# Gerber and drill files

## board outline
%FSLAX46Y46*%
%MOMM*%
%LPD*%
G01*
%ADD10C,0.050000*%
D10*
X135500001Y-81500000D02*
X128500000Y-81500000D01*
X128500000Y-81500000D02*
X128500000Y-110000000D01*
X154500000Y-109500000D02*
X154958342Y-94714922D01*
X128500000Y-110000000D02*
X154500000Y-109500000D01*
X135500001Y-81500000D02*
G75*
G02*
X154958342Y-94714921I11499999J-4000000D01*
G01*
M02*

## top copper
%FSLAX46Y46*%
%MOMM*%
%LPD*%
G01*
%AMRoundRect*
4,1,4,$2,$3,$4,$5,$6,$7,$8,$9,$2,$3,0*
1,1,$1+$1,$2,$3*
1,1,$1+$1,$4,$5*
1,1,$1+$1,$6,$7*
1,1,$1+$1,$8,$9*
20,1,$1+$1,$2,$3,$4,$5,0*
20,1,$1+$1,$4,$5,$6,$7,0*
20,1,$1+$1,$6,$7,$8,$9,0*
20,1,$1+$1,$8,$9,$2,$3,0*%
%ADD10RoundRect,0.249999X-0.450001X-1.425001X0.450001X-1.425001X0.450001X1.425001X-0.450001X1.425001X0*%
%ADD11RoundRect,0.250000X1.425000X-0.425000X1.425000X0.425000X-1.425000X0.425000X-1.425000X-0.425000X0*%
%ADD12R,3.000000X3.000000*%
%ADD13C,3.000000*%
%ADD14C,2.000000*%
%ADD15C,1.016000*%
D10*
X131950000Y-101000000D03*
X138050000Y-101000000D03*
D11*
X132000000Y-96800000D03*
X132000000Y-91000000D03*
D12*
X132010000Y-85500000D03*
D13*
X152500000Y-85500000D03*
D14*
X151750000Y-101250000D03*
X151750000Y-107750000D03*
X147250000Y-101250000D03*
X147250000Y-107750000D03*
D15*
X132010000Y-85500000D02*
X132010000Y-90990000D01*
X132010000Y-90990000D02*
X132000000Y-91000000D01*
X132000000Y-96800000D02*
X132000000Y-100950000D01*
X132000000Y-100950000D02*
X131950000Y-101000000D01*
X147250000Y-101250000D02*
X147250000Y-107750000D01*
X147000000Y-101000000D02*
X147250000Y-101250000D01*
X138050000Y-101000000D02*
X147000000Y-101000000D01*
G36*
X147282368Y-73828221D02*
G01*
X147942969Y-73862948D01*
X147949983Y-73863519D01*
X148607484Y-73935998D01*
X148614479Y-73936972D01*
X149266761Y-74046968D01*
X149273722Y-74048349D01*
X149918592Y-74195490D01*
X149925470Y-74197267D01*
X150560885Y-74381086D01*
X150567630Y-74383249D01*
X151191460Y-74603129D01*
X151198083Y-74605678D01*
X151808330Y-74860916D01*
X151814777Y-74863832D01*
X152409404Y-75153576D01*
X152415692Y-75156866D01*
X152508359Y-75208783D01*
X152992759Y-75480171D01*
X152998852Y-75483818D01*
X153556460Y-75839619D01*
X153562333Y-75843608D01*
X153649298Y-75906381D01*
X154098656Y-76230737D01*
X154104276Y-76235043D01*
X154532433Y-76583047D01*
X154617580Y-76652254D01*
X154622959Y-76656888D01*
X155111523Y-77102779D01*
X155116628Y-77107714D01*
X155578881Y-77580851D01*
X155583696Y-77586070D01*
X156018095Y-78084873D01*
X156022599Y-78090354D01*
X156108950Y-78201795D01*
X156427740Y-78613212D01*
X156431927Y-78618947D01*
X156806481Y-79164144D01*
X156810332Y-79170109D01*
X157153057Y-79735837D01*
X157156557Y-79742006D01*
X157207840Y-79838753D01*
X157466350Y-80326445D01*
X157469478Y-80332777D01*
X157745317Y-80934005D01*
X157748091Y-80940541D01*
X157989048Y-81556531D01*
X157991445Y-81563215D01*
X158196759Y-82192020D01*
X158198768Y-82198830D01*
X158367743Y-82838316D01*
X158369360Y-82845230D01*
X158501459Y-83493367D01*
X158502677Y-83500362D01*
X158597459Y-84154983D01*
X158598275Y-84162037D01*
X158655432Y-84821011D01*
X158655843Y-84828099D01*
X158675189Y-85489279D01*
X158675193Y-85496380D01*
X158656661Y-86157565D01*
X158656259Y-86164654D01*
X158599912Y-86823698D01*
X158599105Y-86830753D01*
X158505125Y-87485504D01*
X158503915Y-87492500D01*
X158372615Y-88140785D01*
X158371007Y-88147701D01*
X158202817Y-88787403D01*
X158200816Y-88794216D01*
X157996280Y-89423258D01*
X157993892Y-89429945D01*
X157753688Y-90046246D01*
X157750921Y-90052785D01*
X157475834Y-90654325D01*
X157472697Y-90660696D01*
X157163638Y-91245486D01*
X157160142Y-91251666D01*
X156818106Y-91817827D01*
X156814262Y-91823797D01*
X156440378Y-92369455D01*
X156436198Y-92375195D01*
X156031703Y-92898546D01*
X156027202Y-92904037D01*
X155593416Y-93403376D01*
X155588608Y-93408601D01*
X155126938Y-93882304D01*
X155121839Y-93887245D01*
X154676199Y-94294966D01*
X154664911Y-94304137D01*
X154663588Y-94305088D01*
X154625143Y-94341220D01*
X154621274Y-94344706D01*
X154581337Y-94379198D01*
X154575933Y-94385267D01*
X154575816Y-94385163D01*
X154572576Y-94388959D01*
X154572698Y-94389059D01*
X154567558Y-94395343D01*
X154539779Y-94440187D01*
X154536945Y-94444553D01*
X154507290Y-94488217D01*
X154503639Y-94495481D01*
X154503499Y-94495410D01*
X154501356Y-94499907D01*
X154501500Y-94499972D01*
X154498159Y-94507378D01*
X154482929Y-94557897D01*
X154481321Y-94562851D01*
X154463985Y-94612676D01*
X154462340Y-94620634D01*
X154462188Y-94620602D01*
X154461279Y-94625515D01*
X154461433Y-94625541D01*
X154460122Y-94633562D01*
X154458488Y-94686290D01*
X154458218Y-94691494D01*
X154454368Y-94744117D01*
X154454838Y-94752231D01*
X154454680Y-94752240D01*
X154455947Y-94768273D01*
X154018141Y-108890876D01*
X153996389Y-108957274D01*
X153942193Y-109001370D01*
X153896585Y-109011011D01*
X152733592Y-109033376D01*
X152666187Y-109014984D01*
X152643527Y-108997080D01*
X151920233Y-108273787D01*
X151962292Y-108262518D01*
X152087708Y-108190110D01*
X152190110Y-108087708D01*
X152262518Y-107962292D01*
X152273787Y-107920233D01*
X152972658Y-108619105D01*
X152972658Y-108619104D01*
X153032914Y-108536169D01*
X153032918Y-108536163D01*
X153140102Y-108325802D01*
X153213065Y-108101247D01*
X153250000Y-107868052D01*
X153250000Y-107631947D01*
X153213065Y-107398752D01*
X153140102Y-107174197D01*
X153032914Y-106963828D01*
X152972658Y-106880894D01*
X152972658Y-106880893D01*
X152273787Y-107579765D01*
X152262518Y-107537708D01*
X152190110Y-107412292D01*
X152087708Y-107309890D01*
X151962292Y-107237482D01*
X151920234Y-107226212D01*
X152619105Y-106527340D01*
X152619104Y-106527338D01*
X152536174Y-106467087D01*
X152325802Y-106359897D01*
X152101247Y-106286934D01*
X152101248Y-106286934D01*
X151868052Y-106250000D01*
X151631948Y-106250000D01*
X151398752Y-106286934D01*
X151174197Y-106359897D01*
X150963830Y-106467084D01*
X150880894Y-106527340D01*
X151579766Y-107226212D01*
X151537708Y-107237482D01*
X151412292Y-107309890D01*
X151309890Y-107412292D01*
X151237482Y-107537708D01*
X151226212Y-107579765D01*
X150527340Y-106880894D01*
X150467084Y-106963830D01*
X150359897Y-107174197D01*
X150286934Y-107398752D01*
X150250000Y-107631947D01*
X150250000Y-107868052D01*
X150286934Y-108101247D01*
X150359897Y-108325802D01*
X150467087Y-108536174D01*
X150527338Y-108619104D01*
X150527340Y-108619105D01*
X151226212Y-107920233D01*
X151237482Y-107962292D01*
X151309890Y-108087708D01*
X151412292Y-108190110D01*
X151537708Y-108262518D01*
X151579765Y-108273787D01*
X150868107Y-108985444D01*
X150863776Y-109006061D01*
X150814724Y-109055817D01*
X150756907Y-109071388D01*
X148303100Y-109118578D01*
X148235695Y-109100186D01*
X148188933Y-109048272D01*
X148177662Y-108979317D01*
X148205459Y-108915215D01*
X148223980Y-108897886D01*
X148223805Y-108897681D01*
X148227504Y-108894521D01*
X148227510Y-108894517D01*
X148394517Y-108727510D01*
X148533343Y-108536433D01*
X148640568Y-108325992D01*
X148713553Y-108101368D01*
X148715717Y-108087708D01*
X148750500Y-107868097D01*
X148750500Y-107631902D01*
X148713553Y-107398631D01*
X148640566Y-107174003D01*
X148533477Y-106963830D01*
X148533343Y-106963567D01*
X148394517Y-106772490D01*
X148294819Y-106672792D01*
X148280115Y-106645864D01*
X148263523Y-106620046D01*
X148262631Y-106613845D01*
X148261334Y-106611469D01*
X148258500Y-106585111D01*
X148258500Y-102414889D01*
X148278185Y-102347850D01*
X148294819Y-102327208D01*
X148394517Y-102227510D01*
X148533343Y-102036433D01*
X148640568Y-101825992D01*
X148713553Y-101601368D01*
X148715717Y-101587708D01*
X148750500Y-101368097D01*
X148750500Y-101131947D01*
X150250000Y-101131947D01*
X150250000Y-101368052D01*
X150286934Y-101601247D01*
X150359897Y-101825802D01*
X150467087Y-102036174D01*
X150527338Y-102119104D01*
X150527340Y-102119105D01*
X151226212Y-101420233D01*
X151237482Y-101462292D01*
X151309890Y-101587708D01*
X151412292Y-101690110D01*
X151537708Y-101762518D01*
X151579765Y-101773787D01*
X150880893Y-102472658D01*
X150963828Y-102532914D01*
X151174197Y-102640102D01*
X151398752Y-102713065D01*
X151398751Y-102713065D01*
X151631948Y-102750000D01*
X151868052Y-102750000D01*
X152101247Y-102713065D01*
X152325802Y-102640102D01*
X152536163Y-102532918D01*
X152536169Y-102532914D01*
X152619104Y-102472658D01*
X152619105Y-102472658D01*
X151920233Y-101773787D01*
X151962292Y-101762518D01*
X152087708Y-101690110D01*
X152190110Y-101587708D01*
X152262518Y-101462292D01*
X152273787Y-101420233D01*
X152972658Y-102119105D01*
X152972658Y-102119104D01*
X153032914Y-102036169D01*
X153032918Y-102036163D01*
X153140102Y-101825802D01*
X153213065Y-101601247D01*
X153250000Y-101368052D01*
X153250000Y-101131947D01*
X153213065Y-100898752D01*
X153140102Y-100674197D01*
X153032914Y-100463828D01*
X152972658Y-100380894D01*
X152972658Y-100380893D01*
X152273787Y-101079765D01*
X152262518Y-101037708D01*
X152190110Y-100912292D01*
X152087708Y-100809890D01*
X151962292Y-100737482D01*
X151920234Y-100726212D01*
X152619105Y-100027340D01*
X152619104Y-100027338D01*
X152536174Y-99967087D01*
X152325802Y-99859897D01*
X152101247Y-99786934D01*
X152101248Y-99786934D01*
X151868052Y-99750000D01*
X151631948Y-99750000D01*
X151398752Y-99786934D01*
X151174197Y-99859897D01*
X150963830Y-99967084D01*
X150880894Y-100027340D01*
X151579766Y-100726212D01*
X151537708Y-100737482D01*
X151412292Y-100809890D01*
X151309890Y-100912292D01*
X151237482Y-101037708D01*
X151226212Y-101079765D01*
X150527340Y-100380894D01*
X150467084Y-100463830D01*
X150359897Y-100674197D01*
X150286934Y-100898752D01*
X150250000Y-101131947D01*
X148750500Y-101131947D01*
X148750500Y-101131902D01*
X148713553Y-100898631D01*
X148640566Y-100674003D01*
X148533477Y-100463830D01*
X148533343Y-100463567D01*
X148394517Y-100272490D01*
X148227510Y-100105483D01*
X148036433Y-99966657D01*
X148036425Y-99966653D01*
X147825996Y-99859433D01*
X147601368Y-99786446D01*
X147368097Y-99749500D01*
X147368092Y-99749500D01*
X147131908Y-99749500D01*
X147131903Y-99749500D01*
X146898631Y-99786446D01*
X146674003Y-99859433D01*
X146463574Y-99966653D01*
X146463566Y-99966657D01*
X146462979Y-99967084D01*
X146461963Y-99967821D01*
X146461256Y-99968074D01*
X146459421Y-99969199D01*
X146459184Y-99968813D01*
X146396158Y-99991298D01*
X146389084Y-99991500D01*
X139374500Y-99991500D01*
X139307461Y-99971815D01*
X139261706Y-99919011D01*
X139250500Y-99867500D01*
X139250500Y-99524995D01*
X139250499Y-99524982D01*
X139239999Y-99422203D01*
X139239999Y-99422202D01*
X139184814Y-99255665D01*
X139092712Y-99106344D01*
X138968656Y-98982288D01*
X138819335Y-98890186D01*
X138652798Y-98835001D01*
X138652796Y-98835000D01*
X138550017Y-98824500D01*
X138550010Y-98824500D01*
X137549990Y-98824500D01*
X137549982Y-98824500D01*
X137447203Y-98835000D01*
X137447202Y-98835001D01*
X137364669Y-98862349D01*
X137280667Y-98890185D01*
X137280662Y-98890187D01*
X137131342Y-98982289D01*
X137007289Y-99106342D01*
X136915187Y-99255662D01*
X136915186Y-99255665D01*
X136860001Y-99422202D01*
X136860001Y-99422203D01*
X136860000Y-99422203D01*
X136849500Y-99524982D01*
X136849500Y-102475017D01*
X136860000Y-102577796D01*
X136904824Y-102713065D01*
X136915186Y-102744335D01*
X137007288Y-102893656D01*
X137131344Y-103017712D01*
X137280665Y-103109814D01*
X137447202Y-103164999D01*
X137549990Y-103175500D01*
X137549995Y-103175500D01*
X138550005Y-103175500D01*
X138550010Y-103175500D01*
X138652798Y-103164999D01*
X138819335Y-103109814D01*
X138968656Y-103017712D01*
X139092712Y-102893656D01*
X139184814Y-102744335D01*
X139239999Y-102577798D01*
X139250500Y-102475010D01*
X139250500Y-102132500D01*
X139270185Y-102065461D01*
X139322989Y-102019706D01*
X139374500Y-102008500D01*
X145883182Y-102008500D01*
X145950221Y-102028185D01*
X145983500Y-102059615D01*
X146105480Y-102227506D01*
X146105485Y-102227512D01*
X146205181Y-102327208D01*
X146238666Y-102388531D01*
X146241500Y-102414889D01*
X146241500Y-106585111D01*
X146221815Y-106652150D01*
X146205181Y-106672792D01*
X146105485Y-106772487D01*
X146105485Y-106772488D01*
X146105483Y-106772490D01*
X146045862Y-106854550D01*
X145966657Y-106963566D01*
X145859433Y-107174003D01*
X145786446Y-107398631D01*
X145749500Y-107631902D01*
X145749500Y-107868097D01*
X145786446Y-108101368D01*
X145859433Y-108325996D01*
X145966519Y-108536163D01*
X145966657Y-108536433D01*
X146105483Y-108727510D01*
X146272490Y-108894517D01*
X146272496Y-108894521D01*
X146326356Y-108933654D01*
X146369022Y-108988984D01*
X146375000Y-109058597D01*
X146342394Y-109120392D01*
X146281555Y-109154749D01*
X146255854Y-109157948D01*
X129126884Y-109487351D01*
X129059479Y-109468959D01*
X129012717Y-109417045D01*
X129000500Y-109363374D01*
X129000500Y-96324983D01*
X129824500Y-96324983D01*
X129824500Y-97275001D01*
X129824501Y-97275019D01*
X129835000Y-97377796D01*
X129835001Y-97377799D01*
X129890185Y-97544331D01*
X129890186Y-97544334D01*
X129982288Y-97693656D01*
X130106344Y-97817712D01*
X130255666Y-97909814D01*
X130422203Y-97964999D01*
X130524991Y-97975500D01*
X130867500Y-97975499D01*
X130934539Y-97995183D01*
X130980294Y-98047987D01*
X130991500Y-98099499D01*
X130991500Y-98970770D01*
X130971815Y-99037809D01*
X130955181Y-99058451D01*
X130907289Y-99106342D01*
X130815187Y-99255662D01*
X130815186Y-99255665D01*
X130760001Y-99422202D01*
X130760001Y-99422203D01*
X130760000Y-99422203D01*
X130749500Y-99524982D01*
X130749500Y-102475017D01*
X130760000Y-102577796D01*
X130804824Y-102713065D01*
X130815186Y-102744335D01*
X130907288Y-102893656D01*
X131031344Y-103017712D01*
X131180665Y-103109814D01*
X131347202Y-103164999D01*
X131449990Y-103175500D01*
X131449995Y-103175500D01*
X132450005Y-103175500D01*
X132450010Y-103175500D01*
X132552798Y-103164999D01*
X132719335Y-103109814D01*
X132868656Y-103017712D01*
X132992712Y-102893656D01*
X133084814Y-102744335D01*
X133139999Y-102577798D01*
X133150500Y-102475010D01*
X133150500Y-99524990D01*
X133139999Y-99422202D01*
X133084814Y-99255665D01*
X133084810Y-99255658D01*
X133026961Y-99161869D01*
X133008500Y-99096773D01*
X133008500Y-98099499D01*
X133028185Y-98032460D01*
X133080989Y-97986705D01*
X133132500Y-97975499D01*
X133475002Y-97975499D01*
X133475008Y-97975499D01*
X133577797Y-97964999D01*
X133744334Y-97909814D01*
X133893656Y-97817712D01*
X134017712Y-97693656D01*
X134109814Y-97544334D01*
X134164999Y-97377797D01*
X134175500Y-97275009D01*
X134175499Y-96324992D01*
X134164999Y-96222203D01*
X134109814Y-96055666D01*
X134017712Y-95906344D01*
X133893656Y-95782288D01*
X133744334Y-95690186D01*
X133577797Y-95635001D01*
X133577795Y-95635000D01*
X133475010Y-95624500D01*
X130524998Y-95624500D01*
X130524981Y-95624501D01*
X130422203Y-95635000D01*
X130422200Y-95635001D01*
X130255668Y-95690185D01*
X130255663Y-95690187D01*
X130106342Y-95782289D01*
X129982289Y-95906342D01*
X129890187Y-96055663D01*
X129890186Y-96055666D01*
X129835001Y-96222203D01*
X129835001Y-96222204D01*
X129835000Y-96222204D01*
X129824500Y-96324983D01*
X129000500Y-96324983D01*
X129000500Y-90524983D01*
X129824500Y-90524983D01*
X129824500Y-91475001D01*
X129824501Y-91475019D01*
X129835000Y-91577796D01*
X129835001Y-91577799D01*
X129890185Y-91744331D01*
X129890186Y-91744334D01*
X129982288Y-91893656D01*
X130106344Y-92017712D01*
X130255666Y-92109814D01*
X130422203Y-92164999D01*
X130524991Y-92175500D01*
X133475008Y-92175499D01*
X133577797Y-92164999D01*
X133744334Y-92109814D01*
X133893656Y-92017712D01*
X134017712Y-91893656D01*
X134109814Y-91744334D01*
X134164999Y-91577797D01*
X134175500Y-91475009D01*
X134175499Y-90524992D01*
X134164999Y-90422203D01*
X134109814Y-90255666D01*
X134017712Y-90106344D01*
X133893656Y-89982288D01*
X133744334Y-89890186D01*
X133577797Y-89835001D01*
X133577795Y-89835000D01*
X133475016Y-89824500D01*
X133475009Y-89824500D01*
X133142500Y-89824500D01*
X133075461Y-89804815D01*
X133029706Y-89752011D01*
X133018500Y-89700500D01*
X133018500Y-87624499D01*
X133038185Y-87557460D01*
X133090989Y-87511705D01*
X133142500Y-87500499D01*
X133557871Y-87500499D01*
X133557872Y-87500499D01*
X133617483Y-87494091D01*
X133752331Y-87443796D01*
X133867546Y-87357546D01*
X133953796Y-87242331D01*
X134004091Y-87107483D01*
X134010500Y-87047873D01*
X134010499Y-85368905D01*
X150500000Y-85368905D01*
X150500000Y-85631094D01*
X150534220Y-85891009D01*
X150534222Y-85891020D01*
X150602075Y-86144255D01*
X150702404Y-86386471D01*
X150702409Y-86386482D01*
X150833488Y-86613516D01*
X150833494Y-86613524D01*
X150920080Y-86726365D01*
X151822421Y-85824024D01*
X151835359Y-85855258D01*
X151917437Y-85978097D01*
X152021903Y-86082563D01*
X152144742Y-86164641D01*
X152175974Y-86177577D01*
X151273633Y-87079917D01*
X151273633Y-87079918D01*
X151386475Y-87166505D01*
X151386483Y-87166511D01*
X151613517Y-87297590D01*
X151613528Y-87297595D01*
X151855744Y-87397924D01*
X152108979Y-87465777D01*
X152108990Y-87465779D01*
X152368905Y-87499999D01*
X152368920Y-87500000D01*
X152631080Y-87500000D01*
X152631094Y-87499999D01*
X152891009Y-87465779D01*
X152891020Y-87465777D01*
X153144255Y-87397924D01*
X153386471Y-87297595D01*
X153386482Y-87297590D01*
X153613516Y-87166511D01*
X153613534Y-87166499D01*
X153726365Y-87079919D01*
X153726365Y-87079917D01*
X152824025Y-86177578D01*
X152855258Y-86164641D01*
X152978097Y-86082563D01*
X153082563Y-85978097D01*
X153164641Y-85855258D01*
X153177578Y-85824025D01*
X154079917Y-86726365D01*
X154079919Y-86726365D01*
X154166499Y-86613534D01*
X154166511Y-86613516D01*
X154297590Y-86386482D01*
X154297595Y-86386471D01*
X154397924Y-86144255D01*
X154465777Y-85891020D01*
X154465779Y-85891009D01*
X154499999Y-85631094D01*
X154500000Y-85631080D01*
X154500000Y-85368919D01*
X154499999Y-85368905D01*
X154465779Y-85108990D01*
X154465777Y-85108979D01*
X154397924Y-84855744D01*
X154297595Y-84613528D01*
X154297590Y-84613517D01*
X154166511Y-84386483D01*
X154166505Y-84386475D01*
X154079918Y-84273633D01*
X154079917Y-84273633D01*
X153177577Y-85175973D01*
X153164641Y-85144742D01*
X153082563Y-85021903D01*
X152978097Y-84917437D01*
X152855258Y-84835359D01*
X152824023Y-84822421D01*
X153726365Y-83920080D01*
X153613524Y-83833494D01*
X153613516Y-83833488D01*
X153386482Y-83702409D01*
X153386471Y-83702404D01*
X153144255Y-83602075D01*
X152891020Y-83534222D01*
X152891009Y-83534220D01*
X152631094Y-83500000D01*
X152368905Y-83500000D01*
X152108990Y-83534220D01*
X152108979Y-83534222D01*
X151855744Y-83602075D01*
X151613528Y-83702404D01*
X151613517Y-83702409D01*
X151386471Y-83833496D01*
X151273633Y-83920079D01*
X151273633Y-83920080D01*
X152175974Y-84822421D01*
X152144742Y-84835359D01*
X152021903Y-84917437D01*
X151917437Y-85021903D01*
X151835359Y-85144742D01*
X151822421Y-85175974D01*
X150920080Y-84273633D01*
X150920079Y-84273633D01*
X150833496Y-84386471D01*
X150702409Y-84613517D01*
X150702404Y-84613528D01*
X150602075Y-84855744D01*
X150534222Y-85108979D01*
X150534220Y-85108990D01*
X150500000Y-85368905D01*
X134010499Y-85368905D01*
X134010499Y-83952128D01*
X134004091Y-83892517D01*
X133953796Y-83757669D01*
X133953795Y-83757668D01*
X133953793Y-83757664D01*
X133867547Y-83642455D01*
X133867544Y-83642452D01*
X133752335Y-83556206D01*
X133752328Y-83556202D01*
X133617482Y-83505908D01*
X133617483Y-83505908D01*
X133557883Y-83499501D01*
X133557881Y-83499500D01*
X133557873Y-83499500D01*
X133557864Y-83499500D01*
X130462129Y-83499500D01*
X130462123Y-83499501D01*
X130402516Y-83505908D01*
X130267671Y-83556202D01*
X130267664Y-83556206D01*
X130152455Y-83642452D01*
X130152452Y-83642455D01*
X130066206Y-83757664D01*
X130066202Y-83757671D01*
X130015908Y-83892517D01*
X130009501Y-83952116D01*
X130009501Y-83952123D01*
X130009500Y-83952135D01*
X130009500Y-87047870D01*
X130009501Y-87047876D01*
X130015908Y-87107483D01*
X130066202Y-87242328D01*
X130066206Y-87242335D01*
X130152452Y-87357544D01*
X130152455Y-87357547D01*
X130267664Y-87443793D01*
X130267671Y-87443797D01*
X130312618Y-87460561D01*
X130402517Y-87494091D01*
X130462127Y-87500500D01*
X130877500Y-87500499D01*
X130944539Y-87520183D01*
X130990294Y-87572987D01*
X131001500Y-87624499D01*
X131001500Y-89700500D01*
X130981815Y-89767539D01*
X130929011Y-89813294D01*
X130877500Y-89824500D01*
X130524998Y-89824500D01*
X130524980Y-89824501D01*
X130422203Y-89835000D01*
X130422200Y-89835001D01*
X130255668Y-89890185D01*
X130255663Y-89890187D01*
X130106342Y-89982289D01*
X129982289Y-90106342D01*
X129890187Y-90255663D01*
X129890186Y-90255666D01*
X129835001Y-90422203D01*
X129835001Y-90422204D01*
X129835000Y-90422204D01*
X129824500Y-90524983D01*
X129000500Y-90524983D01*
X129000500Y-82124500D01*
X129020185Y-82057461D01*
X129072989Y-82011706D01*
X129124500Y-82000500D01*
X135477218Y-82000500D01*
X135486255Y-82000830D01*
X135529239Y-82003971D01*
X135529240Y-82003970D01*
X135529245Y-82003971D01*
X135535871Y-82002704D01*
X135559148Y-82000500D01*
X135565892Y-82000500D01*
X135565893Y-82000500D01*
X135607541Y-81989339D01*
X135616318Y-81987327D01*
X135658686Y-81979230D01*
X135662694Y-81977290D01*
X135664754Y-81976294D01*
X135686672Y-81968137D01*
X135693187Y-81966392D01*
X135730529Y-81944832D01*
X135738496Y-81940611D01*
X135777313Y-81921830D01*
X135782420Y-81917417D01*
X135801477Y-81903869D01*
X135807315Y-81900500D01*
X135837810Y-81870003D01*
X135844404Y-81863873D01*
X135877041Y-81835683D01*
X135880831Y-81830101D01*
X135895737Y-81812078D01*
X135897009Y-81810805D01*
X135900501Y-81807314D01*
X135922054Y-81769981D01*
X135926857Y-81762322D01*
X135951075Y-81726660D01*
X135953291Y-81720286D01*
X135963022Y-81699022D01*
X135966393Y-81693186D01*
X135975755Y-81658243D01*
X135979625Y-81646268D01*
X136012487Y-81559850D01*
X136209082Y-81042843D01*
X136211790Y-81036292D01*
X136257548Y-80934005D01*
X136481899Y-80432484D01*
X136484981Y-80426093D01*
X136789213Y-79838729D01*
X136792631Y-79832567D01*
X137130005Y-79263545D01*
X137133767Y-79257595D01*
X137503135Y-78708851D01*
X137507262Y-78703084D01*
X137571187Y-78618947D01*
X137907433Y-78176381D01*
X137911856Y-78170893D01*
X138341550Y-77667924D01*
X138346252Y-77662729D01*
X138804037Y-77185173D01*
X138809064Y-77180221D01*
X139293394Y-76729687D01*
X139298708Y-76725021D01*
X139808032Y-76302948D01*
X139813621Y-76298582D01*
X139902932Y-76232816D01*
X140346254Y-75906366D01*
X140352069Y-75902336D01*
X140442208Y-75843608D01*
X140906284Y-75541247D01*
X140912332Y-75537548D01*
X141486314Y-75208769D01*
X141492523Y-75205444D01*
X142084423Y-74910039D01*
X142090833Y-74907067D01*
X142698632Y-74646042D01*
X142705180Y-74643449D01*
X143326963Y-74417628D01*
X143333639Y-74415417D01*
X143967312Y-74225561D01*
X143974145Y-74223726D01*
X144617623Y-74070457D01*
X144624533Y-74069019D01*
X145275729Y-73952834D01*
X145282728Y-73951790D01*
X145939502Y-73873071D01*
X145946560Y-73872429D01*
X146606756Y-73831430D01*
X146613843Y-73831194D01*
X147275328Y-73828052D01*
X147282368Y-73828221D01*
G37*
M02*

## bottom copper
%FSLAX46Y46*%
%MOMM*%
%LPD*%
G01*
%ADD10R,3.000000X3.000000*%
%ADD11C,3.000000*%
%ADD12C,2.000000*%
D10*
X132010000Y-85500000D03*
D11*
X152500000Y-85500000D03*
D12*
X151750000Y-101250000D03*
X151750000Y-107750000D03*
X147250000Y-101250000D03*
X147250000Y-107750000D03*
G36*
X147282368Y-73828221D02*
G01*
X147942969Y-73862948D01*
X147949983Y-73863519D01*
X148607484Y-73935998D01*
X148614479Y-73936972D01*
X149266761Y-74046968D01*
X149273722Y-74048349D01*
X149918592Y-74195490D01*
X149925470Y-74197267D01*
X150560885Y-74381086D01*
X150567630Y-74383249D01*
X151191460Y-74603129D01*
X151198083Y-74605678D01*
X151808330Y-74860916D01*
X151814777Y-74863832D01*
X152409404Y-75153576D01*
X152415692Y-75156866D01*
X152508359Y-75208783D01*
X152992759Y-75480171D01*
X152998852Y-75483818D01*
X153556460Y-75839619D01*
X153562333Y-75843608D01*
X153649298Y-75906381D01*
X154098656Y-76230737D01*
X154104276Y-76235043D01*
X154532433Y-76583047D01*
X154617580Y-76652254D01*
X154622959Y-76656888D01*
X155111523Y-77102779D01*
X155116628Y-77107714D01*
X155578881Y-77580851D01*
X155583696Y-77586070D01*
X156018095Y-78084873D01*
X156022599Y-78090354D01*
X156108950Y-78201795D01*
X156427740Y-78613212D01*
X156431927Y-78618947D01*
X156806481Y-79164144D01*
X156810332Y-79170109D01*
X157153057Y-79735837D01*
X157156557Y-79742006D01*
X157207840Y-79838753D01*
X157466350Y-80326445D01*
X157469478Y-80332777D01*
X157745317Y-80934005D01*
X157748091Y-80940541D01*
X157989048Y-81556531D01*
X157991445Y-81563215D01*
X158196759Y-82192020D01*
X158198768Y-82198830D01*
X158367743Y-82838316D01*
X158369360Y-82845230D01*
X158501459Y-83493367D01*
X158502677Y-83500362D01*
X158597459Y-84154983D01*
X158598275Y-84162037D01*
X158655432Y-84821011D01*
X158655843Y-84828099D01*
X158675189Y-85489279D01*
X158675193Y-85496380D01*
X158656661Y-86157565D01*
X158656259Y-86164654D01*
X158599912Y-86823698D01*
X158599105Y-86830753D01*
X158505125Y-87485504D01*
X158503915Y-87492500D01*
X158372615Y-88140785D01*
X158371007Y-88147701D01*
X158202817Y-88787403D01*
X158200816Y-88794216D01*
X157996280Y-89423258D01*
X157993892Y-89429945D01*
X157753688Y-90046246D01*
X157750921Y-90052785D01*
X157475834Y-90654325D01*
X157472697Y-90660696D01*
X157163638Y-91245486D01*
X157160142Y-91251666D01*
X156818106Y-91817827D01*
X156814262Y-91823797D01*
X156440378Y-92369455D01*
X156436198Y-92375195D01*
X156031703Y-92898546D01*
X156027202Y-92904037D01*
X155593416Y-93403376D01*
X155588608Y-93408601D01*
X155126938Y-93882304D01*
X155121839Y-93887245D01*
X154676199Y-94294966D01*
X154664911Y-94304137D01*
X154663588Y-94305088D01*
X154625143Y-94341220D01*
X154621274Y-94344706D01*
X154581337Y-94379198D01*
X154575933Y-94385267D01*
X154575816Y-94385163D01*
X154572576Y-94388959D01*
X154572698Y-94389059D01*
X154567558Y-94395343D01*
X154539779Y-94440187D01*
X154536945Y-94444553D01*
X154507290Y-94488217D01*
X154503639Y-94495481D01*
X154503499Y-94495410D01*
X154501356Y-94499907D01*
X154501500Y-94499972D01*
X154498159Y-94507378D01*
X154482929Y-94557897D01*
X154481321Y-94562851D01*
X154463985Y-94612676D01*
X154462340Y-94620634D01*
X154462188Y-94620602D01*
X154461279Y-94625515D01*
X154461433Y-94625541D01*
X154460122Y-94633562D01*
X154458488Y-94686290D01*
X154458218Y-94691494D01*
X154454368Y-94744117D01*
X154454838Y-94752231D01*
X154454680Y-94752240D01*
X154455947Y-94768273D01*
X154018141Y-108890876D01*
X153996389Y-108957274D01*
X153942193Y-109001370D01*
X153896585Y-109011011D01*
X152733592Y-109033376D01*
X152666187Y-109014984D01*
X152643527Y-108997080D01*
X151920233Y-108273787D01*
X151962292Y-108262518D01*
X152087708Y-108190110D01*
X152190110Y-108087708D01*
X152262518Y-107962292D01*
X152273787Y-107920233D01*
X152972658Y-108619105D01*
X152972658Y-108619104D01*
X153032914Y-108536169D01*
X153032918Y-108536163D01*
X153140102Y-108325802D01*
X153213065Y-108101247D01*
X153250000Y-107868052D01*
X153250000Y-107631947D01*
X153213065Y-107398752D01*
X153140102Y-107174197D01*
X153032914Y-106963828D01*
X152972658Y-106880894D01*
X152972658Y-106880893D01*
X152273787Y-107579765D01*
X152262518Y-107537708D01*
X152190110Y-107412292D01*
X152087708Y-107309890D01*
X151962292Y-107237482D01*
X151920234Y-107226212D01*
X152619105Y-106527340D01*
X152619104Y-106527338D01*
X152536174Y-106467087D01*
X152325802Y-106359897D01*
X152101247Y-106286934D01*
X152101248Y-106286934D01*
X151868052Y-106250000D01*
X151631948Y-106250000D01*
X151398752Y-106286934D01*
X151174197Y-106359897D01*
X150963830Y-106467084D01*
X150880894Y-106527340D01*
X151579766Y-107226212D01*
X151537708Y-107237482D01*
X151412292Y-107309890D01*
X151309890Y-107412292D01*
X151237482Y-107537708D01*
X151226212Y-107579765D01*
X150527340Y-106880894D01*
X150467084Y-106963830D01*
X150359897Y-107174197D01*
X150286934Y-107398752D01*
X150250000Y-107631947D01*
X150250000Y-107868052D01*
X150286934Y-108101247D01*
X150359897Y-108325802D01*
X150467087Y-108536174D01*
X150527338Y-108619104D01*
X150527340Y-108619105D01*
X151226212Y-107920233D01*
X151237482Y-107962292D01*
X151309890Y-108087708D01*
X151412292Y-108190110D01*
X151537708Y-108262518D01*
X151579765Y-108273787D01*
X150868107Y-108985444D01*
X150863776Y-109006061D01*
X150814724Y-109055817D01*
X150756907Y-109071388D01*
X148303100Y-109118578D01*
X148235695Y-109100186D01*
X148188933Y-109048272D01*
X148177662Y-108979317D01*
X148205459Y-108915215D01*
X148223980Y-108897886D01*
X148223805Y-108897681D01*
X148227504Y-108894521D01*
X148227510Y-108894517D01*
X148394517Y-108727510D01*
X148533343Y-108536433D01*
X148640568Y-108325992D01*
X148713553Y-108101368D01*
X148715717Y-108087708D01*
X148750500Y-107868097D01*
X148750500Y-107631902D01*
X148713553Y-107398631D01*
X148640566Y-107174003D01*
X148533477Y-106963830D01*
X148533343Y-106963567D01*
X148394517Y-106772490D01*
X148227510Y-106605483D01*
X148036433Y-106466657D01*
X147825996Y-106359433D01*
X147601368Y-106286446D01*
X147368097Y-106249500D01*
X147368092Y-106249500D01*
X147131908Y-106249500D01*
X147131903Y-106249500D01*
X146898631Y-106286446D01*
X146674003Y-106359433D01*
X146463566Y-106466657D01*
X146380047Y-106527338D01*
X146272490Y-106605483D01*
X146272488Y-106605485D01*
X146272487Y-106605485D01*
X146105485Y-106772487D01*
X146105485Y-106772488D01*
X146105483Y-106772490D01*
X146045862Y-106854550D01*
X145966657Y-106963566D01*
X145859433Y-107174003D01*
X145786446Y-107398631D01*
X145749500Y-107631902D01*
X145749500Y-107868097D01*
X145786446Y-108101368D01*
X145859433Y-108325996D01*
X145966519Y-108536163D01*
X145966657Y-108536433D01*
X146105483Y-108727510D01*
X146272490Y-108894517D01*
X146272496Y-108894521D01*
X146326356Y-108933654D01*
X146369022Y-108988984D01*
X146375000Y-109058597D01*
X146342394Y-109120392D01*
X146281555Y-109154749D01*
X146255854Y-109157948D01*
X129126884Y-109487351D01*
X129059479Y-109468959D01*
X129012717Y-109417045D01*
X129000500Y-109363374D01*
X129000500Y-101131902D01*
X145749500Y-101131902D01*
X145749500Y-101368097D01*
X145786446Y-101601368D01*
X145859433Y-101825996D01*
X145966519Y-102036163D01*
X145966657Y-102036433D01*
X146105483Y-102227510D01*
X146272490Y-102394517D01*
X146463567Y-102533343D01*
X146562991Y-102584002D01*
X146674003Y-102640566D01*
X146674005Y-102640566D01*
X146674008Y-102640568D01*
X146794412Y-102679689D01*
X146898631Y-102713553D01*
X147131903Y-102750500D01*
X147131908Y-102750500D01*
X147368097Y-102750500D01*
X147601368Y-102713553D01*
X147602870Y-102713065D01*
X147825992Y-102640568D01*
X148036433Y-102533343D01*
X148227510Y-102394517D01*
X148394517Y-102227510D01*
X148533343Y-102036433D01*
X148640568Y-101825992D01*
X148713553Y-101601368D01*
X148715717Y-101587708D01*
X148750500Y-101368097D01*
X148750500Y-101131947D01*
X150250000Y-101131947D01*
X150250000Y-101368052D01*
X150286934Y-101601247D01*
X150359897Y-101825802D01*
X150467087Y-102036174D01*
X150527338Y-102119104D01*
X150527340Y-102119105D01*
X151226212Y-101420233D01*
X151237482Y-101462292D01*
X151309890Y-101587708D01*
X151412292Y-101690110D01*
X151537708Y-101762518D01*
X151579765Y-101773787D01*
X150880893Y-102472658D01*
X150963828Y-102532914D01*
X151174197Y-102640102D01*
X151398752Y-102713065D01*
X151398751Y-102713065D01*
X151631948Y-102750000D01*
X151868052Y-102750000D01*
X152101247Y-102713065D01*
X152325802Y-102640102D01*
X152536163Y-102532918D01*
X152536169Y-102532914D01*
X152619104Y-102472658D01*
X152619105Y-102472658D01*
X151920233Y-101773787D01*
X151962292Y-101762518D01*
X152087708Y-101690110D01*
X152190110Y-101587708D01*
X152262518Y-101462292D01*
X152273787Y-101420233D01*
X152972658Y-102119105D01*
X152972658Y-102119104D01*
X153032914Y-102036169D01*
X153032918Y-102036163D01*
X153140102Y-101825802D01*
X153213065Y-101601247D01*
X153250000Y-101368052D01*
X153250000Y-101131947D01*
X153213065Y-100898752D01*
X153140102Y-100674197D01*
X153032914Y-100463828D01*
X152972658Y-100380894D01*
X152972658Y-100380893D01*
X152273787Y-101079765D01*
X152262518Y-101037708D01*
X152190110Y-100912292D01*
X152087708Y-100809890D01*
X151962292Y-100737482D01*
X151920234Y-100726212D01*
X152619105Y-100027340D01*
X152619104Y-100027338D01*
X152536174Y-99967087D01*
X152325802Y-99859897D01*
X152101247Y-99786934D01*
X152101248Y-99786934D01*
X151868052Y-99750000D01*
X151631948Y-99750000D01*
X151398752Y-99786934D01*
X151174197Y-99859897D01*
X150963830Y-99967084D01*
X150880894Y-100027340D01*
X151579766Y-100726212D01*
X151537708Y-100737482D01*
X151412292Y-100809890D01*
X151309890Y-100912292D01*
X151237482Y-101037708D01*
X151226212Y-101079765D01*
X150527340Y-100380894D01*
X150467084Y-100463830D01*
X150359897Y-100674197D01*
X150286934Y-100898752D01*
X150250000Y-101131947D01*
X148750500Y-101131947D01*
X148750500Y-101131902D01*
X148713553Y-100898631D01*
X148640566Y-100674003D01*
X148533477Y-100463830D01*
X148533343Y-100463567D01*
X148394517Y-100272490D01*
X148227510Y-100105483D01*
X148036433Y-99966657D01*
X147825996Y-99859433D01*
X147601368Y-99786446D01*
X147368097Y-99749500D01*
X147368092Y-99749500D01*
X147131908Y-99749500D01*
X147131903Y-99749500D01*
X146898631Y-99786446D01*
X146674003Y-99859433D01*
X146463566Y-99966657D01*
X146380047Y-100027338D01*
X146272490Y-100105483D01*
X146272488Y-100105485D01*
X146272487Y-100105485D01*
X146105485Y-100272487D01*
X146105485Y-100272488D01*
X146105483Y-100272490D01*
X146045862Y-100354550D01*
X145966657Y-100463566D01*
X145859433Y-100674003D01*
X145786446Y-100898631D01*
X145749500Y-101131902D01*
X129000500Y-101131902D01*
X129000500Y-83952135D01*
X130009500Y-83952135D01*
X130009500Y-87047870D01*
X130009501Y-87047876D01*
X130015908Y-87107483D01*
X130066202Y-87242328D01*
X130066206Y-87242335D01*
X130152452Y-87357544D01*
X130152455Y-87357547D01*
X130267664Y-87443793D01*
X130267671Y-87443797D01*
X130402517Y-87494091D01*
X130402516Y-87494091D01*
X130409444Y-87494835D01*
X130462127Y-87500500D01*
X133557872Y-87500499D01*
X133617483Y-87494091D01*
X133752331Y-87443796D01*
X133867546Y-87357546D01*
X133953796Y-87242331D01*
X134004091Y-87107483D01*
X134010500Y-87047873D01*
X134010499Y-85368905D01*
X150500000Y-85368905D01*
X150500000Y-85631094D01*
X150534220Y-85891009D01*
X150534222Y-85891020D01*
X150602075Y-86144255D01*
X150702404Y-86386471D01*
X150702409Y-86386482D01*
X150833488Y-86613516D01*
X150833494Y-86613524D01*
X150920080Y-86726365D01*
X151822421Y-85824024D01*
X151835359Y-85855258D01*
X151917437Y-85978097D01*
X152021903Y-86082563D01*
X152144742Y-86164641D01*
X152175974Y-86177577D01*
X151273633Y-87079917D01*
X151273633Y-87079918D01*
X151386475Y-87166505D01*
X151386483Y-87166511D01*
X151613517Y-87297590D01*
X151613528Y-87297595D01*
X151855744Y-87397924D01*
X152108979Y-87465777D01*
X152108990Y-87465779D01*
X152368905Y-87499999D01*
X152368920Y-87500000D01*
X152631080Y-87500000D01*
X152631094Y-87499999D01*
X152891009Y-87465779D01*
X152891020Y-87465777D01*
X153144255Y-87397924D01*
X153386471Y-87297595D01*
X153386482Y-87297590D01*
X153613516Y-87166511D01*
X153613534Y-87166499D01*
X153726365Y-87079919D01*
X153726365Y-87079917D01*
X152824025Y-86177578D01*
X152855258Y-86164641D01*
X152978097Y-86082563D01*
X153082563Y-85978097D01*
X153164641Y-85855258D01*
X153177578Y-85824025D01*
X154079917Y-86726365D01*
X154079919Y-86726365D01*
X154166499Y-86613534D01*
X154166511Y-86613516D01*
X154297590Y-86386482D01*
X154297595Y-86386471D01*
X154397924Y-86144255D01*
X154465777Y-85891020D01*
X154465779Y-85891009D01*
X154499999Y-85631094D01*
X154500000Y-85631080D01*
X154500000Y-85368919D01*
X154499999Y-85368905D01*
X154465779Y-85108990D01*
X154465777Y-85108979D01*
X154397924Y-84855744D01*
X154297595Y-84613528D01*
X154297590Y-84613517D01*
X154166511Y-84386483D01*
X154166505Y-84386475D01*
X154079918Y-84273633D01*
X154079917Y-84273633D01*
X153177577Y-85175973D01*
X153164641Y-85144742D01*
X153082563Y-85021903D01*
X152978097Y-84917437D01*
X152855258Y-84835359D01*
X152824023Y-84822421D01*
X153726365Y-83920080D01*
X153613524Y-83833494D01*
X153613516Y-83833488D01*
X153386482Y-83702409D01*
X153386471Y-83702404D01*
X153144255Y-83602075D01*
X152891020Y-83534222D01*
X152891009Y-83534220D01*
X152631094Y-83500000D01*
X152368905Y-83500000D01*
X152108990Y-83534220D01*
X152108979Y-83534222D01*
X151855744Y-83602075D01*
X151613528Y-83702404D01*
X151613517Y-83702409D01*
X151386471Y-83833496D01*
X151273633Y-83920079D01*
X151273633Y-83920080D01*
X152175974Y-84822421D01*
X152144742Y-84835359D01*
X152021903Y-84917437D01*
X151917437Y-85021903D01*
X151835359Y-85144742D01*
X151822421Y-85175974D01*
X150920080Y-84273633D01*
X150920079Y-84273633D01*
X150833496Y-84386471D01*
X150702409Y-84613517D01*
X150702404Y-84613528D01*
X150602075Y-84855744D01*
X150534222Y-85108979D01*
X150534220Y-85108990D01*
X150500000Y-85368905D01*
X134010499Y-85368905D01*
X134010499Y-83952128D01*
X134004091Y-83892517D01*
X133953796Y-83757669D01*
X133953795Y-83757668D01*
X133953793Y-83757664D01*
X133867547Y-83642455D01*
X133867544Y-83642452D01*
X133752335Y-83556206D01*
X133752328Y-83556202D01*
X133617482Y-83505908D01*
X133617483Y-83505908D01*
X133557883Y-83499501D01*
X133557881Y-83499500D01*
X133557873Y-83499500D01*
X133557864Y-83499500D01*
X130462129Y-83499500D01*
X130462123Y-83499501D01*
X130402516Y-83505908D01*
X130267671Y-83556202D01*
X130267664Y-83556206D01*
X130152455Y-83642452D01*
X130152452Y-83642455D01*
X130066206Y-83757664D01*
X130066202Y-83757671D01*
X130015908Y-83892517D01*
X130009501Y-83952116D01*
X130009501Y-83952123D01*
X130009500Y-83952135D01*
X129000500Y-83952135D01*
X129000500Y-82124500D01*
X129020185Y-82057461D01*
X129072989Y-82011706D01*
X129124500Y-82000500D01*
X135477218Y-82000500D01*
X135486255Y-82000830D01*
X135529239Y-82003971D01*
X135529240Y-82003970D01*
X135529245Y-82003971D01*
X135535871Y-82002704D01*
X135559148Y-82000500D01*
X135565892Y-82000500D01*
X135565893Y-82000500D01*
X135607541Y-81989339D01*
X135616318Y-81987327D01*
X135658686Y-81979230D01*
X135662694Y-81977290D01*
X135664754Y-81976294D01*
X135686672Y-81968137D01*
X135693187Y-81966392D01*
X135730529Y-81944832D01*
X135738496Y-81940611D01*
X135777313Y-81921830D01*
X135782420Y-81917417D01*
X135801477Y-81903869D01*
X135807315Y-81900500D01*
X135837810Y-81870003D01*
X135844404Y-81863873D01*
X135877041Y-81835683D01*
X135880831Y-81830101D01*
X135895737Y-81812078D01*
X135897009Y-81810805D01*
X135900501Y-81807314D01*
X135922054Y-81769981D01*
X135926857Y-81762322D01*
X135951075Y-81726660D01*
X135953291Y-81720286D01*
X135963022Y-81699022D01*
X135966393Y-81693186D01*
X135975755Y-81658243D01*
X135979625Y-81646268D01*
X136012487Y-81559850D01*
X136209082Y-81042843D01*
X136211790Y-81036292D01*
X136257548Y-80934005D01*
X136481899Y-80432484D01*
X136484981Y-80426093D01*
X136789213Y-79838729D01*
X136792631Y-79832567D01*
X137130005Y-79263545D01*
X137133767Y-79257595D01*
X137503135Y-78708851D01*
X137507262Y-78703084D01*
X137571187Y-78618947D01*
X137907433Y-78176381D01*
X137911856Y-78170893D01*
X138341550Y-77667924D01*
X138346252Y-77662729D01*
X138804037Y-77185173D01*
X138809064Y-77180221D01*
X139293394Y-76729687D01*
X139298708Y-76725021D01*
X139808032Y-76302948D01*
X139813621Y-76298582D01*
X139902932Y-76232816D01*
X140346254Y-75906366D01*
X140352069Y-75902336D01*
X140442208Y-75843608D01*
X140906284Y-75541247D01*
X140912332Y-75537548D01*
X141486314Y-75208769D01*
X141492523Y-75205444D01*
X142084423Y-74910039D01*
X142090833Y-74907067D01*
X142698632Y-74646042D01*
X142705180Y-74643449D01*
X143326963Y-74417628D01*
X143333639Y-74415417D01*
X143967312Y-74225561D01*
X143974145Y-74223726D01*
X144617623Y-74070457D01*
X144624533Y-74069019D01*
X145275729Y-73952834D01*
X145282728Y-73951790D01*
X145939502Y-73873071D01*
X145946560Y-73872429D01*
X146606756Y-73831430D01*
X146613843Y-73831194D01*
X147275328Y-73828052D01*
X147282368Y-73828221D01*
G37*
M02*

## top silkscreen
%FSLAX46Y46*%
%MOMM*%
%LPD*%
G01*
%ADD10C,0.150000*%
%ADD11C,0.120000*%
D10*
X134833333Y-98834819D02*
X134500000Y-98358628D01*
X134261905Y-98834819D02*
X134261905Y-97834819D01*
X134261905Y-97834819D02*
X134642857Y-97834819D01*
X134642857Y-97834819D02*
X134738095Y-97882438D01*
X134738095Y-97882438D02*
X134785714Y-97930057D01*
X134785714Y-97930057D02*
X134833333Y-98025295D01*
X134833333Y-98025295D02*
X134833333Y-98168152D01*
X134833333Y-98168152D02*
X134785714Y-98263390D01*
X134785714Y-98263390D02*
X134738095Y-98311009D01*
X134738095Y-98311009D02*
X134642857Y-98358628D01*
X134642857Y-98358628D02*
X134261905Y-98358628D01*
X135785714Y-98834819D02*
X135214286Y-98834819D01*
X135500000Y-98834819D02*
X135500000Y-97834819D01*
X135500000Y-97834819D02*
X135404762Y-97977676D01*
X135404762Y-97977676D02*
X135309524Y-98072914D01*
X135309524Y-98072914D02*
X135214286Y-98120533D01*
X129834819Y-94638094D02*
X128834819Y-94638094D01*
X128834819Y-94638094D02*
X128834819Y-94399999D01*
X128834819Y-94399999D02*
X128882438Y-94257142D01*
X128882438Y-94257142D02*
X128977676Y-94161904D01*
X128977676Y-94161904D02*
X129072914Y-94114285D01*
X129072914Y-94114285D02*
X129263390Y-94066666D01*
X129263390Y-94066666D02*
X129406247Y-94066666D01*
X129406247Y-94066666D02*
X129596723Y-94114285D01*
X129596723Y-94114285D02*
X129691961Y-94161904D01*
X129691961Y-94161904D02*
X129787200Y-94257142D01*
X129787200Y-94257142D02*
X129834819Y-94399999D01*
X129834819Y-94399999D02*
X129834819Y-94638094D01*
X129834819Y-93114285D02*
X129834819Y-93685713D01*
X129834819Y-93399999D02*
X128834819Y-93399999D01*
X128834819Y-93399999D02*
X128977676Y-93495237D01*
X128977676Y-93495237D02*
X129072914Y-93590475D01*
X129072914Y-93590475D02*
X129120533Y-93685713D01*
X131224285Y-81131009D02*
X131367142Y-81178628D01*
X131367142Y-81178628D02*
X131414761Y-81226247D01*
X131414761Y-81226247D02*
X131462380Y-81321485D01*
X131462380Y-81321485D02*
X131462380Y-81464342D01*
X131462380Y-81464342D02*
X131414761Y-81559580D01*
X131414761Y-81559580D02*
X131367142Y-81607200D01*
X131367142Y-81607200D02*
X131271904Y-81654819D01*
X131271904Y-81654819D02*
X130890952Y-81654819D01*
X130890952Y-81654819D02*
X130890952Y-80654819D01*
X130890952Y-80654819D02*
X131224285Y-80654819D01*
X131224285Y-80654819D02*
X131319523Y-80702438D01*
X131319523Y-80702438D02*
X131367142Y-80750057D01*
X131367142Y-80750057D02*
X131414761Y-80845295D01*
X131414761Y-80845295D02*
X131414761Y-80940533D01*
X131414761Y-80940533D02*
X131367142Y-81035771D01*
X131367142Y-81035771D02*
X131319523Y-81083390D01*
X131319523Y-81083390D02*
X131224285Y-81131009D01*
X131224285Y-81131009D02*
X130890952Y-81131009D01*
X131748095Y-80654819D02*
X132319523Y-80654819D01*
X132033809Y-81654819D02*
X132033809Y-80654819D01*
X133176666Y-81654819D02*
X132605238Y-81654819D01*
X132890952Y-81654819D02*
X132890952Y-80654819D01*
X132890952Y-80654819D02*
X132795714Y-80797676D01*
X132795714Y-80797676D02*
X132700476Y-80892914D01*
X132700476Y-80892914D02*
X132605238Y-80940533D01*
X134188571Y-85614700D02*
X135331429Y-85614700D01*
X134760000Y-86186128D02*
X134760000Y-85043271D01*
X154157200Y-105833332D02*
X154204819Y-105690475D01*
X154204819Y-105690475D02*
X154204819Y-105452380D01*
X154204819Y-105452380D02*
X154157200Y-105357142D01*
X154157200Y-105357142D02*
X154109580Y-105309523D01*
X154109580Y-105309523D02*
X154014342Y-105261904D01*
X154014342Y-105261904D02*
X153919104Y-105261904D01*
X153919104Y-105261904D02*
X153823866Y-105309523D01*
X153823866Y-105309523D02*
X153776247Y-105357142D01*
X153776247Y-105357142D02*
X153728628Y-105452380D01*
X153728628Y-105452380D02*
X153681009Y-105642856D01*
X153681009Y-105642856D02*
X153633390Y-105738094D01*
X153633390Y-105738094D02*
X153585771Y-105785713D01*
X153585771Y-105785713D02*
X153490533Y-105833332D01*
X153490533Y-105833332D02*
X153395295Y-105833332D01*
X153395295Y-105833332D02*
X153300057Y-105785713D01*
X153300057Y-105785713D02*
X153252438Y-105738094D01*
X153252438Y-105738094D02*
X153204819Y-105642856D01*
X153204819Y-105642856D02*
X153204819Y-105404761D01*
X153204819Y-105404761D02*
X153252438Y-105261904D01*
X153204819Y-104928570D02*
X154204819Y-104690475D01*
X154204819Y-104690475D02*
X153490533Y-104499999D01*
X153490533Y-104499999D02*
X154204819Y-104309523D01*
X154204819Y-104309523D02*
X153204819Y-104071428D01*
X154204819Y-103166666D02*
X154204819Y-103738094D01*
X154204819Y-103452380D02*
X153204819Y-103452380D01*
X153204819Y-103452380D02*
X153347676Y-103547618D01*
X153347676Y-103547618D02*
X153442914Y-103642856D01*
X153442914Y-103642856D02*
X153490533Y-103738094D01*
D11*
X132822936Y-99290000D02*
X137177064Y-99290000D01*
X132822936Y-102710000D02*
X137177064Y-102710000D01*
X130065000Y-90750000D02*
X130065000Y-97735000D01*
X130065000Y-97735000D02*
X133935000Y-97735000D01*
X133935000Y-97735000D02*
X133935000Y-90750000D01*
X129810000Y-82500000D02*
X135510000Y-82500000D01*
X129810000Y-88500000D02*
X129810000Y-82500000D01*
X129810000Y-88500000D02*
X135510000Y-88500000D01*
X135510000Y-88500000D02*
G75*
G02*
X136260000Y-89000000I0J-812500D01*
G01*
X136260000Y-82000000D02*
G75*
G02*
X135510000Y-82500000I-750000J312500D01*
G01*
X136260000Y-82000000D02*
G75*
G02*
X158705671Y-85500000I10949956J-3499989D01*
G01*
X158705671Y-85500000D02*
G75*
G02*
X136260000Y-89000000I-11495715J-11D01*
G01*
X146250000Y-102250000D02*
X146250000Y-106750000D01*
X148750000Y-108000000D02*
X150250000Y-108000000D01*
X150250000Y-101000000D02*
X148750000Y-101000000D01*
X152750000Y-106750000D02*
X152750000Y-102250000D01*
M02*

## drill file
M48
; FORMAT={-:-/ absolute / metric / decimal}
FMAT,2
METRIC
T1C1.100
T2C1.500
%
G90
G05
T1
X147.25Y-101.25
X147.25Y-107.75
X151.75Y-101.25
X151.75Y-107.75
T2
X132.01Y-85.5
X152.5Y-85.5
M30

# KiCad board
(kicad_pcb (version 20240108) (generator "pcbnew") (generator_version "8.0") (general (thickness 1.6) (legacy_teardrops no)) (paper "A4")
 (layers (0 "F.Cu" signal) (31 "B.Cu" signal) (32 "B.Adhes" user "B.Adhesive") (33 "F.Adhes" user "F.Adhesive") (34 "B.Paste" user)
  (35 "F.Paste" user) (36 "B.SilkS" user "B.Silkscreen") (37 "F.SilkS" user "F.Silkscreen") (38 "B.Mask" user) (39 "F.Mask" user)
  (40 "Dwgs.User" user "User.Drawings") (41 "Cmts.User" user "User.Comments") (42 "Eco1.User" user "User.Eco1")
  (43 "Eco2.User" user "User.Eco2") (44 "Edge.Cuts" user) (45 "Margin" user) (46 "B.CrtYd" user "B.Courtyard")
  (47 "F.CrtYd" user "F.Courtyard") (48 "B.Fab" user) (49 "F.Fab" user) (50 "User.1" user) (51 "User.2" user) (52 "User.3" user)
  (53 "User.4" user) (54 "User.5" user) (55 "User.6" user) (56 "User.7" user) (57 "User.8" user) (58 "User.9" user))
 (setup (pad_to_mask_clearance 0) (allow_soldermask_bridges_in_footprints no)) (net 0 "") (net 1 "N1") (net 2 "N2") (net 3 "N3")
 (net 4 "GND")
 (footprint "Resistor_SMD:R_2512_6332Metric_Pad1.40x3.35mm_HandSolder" (layer "F.Cu") (at 135 101)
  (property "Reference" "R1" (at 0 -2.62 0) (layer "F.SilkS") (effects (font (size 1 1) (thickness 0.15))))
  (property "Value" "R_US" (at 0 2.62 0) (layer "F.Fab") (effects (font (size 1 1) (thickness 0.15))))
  (fp_line (start -2.177064 -1.71) (end 2.177064 -1.71) (stroke (width 0.12) (type solid)) (layer "F.SilkS"))
  (fp_line (start -2.177064 1.71) (end 2.177064 1.71) (stroke (width 0.12) (type solid)) (layer "F.SilkS"))
  (pad "1" smd roundrect (at -3.05 0) (size 1.4 3.35) (layers "F.Cu" "F.Paste" "F.Mask") (roundrect_rratio 0.178571) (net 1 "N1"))
  (pad "2" smd roundrect (at 3.05 0) (size 1.4 3.35) (layers "F.Cu" "F.Paste" "F.Mask") (roundrect_rratio 0.178571) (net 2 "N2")))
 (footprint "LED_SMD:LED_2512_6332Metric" (layer "F.Cu") (at 132 93.9 90)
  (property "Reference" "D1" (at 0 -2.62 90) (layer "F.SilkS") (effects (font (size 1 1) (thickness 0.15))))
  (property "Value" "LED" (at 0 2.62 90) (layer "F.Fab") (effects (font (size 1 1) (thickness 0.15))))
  (fp_line (start 3.15 -1.935) (end -3.835 -1.935) (stroke (width 0.12) (type solid)) (layer "F.SilkS"))
  (fp_line (start -3.835 -1.935) (end -3.835 1.935) (stroke (width 0.12) (type solid)) (layer "F.SilkS"))
  (fp_line (start -3.835 1.935) (end 3.15 1.935) (stroke (width 0.12) (type solid)) (layer "F.SilkS"))
  (pad "1" smd roundrect (at -2.9 0 90) (size 1.35 3.35) (layers "F.Cu" "F.Paste" "F.Mask") (roundrect_rratio 0.185185) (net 1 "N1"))
  (pad "2" smd roundrect (at 2.9 0 90) (size 1.35 3.35) (layers "F.Cu" "F.Paste" "F.Mask") (roundrect_rratio 0.185185) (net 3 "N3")))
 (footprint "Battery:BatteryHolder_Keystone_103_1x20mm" (layer "F.Cu") (at 132.01 85.5)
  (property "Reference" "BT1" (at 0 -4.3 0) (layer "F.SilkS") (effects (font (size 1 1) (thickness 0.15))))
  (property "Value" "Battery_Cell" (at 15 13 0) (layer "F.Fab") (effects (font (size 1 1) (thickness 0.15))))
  (fp_line (start -2.2 -3) (end 3.5 -3) (stroke (width 0.12) (type solid)) (layer "F.SilkS"))
  (fp_line (start -2.2 3) (end -2.2 -3) (stroke (width 0.12) (type solid)) (layer "F.SilkS"))
  (fp_line (start -2.2 3) (end 3.5 3) (stroke (width 0.12) (type solid)) (layer "F.SilkS"))
  (fp_arc (start 3.5 3) (mid 3.950694 3.136459) (end 4.25 3.5) (stroke (width 0.12) (type solid)) (layer "F.SilkS"))
  (fp_arc (start 4.25 -3.5) (mid 3.950694 -3.136459) (end 3.5 -3) (stroke (width 0.12) (type solid)) (layer "F.SilkS"))
  (fp_arc (start 4.25 -3.5) (mid 16.971103 -11.358466) (end 26.695671 0) (stroke (width 0.12) (type solid)) (layer "F.SilkS"))
  (fp_arc (start 26.695671 0) (mid 16.971103 11.358466) (end 4.25 3.5) (stroke (width 0.12) (type solid)) (layer "F.SilkS"))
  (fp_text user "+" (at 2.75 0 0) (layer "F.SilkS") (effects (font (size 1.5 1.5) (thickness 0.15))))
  (pad "1" thru_hole rect (at 0 0) (size 3 3) (drill 1.5) (layers "*.Cu" "*.Mask") (remove_unused_layers no) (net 3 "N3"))
  (pad "2" thru_hole circle (at 20.49 0) (size 3 3) (drill 1.5) (layers "*.Cu" "*.Mask") (remove_unused_layers no) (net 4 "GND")))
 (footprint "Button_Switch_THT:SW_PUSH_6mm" (layer "F.Cu") (at 151.75 101.25 -90)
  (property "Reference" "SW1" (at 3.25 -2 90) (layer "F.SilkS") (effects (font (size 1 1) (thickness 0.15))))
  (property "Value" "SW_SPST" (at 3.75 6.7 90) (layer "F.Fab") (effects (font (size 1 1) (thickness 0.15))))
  (fp_line (start 1 5.5) (end 5.5 5.5) (stroke (width 0.12) (type solid)) (layer "F.SilkS"))
  (fp_line (start 6.75 3) (end 6.75 1.5) (stroke (width 0.12) (type solid)) (layer "F.SilkS"))
  (fp_line (start -0.25 1.5) (end -0.25 3) (stroke (width 0.12) (type solid)) (layer "F.SilkS"))
  (fp_line (start 5.5 -1) (end 1 -1) (stroke (width 0.12) (type solid)) (layer "F.SilkS"))
  (pad "1" thru_hole circle (at 0 0) (size 2 2) (drill 1.1) (layers "*.Cu" "*.Mask") (remove_unused_layers no) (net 4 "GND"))
  (pad "1" thru_hole circle (at 6.5 0) (size 2 2) (drill 1.1) (layers "*.Cu" "*.Mask") (remove_unused_layers no) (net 4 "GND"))
  (pad "2" thru_hole circle (at 0 4.5) (size 2 2) (drill 1.1) (layers "*.Cu" "*.Mask") (remove_unused_layers no) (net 2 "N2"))
  (pad "2" thru_hole circle (at 6.5 4.5) (size 2 2) (drill 1.1) (layers "*.Cu" "*.Mask") (remove_unused_layers no) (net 2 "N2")))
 (gr_line (start 135.500001 81.5) (end 128.5 81.5) (stroke (width 0.05) (type default)) (layer "Edge.Cuts"))
 (gr_line (start 128.5 81.5) (end 128.5 110) (stroke (width 0.05) (type default)) (layer "Edge.Cuts"))
 (gr_line (start 154.5 109.5) (end 154.958342 94.714922) (stroke (width 0.05) (type default)) (layer "Edge.Cuts"))
 (gr_line (start 128.5 110) (end 154.5 109.5) (stroke (width 0.05) (type default)) (layer "Edge.Cuts"))
 (gr_arc (start 135.500001 81.5) (mid 153.840641 75.427483) (end 154.958342 94.714922) (stroke (width 0.05) (type default))
  (layer "Edge.Cuts"))
 (segment (start 132.01 85.5) (end 132.01 90.99) (width 1.016) (layer "F.Cu") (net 3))
 (segment (start 132.01 90.99) (end 132 91) (width 1.016) (layer "F.Cu") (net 3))
 (segment (start 132 96.8) (end 132 100.95) (width 1.016) (layer "F.Cu") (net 1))
 (segment (start 132 100.95) (end 131.95 101) (width 1.016) (layer "F.Cu") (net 1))
 (segment (start 147.25 101.25) (end 147.25 107.75) (width 1.016) (layer "F.Cu") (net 2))
 (segment (start 147 101) (end 147.25 101.25) (width 1.016) (layer "F.Cu") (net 2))
 (segment (start 138.05 101) (end 147 101) (width 1.016) (layer "F.Cu") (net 2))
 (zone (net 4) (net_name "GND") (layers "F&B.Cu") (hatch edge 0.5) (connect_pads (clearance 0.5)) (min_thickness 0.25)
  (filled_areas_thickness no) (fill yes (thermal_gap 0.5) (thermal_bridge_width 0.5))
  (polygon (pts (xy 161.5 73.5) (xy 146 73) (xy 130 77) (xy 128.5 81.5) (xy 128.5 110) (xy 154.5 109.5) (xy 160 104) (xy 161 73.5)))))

